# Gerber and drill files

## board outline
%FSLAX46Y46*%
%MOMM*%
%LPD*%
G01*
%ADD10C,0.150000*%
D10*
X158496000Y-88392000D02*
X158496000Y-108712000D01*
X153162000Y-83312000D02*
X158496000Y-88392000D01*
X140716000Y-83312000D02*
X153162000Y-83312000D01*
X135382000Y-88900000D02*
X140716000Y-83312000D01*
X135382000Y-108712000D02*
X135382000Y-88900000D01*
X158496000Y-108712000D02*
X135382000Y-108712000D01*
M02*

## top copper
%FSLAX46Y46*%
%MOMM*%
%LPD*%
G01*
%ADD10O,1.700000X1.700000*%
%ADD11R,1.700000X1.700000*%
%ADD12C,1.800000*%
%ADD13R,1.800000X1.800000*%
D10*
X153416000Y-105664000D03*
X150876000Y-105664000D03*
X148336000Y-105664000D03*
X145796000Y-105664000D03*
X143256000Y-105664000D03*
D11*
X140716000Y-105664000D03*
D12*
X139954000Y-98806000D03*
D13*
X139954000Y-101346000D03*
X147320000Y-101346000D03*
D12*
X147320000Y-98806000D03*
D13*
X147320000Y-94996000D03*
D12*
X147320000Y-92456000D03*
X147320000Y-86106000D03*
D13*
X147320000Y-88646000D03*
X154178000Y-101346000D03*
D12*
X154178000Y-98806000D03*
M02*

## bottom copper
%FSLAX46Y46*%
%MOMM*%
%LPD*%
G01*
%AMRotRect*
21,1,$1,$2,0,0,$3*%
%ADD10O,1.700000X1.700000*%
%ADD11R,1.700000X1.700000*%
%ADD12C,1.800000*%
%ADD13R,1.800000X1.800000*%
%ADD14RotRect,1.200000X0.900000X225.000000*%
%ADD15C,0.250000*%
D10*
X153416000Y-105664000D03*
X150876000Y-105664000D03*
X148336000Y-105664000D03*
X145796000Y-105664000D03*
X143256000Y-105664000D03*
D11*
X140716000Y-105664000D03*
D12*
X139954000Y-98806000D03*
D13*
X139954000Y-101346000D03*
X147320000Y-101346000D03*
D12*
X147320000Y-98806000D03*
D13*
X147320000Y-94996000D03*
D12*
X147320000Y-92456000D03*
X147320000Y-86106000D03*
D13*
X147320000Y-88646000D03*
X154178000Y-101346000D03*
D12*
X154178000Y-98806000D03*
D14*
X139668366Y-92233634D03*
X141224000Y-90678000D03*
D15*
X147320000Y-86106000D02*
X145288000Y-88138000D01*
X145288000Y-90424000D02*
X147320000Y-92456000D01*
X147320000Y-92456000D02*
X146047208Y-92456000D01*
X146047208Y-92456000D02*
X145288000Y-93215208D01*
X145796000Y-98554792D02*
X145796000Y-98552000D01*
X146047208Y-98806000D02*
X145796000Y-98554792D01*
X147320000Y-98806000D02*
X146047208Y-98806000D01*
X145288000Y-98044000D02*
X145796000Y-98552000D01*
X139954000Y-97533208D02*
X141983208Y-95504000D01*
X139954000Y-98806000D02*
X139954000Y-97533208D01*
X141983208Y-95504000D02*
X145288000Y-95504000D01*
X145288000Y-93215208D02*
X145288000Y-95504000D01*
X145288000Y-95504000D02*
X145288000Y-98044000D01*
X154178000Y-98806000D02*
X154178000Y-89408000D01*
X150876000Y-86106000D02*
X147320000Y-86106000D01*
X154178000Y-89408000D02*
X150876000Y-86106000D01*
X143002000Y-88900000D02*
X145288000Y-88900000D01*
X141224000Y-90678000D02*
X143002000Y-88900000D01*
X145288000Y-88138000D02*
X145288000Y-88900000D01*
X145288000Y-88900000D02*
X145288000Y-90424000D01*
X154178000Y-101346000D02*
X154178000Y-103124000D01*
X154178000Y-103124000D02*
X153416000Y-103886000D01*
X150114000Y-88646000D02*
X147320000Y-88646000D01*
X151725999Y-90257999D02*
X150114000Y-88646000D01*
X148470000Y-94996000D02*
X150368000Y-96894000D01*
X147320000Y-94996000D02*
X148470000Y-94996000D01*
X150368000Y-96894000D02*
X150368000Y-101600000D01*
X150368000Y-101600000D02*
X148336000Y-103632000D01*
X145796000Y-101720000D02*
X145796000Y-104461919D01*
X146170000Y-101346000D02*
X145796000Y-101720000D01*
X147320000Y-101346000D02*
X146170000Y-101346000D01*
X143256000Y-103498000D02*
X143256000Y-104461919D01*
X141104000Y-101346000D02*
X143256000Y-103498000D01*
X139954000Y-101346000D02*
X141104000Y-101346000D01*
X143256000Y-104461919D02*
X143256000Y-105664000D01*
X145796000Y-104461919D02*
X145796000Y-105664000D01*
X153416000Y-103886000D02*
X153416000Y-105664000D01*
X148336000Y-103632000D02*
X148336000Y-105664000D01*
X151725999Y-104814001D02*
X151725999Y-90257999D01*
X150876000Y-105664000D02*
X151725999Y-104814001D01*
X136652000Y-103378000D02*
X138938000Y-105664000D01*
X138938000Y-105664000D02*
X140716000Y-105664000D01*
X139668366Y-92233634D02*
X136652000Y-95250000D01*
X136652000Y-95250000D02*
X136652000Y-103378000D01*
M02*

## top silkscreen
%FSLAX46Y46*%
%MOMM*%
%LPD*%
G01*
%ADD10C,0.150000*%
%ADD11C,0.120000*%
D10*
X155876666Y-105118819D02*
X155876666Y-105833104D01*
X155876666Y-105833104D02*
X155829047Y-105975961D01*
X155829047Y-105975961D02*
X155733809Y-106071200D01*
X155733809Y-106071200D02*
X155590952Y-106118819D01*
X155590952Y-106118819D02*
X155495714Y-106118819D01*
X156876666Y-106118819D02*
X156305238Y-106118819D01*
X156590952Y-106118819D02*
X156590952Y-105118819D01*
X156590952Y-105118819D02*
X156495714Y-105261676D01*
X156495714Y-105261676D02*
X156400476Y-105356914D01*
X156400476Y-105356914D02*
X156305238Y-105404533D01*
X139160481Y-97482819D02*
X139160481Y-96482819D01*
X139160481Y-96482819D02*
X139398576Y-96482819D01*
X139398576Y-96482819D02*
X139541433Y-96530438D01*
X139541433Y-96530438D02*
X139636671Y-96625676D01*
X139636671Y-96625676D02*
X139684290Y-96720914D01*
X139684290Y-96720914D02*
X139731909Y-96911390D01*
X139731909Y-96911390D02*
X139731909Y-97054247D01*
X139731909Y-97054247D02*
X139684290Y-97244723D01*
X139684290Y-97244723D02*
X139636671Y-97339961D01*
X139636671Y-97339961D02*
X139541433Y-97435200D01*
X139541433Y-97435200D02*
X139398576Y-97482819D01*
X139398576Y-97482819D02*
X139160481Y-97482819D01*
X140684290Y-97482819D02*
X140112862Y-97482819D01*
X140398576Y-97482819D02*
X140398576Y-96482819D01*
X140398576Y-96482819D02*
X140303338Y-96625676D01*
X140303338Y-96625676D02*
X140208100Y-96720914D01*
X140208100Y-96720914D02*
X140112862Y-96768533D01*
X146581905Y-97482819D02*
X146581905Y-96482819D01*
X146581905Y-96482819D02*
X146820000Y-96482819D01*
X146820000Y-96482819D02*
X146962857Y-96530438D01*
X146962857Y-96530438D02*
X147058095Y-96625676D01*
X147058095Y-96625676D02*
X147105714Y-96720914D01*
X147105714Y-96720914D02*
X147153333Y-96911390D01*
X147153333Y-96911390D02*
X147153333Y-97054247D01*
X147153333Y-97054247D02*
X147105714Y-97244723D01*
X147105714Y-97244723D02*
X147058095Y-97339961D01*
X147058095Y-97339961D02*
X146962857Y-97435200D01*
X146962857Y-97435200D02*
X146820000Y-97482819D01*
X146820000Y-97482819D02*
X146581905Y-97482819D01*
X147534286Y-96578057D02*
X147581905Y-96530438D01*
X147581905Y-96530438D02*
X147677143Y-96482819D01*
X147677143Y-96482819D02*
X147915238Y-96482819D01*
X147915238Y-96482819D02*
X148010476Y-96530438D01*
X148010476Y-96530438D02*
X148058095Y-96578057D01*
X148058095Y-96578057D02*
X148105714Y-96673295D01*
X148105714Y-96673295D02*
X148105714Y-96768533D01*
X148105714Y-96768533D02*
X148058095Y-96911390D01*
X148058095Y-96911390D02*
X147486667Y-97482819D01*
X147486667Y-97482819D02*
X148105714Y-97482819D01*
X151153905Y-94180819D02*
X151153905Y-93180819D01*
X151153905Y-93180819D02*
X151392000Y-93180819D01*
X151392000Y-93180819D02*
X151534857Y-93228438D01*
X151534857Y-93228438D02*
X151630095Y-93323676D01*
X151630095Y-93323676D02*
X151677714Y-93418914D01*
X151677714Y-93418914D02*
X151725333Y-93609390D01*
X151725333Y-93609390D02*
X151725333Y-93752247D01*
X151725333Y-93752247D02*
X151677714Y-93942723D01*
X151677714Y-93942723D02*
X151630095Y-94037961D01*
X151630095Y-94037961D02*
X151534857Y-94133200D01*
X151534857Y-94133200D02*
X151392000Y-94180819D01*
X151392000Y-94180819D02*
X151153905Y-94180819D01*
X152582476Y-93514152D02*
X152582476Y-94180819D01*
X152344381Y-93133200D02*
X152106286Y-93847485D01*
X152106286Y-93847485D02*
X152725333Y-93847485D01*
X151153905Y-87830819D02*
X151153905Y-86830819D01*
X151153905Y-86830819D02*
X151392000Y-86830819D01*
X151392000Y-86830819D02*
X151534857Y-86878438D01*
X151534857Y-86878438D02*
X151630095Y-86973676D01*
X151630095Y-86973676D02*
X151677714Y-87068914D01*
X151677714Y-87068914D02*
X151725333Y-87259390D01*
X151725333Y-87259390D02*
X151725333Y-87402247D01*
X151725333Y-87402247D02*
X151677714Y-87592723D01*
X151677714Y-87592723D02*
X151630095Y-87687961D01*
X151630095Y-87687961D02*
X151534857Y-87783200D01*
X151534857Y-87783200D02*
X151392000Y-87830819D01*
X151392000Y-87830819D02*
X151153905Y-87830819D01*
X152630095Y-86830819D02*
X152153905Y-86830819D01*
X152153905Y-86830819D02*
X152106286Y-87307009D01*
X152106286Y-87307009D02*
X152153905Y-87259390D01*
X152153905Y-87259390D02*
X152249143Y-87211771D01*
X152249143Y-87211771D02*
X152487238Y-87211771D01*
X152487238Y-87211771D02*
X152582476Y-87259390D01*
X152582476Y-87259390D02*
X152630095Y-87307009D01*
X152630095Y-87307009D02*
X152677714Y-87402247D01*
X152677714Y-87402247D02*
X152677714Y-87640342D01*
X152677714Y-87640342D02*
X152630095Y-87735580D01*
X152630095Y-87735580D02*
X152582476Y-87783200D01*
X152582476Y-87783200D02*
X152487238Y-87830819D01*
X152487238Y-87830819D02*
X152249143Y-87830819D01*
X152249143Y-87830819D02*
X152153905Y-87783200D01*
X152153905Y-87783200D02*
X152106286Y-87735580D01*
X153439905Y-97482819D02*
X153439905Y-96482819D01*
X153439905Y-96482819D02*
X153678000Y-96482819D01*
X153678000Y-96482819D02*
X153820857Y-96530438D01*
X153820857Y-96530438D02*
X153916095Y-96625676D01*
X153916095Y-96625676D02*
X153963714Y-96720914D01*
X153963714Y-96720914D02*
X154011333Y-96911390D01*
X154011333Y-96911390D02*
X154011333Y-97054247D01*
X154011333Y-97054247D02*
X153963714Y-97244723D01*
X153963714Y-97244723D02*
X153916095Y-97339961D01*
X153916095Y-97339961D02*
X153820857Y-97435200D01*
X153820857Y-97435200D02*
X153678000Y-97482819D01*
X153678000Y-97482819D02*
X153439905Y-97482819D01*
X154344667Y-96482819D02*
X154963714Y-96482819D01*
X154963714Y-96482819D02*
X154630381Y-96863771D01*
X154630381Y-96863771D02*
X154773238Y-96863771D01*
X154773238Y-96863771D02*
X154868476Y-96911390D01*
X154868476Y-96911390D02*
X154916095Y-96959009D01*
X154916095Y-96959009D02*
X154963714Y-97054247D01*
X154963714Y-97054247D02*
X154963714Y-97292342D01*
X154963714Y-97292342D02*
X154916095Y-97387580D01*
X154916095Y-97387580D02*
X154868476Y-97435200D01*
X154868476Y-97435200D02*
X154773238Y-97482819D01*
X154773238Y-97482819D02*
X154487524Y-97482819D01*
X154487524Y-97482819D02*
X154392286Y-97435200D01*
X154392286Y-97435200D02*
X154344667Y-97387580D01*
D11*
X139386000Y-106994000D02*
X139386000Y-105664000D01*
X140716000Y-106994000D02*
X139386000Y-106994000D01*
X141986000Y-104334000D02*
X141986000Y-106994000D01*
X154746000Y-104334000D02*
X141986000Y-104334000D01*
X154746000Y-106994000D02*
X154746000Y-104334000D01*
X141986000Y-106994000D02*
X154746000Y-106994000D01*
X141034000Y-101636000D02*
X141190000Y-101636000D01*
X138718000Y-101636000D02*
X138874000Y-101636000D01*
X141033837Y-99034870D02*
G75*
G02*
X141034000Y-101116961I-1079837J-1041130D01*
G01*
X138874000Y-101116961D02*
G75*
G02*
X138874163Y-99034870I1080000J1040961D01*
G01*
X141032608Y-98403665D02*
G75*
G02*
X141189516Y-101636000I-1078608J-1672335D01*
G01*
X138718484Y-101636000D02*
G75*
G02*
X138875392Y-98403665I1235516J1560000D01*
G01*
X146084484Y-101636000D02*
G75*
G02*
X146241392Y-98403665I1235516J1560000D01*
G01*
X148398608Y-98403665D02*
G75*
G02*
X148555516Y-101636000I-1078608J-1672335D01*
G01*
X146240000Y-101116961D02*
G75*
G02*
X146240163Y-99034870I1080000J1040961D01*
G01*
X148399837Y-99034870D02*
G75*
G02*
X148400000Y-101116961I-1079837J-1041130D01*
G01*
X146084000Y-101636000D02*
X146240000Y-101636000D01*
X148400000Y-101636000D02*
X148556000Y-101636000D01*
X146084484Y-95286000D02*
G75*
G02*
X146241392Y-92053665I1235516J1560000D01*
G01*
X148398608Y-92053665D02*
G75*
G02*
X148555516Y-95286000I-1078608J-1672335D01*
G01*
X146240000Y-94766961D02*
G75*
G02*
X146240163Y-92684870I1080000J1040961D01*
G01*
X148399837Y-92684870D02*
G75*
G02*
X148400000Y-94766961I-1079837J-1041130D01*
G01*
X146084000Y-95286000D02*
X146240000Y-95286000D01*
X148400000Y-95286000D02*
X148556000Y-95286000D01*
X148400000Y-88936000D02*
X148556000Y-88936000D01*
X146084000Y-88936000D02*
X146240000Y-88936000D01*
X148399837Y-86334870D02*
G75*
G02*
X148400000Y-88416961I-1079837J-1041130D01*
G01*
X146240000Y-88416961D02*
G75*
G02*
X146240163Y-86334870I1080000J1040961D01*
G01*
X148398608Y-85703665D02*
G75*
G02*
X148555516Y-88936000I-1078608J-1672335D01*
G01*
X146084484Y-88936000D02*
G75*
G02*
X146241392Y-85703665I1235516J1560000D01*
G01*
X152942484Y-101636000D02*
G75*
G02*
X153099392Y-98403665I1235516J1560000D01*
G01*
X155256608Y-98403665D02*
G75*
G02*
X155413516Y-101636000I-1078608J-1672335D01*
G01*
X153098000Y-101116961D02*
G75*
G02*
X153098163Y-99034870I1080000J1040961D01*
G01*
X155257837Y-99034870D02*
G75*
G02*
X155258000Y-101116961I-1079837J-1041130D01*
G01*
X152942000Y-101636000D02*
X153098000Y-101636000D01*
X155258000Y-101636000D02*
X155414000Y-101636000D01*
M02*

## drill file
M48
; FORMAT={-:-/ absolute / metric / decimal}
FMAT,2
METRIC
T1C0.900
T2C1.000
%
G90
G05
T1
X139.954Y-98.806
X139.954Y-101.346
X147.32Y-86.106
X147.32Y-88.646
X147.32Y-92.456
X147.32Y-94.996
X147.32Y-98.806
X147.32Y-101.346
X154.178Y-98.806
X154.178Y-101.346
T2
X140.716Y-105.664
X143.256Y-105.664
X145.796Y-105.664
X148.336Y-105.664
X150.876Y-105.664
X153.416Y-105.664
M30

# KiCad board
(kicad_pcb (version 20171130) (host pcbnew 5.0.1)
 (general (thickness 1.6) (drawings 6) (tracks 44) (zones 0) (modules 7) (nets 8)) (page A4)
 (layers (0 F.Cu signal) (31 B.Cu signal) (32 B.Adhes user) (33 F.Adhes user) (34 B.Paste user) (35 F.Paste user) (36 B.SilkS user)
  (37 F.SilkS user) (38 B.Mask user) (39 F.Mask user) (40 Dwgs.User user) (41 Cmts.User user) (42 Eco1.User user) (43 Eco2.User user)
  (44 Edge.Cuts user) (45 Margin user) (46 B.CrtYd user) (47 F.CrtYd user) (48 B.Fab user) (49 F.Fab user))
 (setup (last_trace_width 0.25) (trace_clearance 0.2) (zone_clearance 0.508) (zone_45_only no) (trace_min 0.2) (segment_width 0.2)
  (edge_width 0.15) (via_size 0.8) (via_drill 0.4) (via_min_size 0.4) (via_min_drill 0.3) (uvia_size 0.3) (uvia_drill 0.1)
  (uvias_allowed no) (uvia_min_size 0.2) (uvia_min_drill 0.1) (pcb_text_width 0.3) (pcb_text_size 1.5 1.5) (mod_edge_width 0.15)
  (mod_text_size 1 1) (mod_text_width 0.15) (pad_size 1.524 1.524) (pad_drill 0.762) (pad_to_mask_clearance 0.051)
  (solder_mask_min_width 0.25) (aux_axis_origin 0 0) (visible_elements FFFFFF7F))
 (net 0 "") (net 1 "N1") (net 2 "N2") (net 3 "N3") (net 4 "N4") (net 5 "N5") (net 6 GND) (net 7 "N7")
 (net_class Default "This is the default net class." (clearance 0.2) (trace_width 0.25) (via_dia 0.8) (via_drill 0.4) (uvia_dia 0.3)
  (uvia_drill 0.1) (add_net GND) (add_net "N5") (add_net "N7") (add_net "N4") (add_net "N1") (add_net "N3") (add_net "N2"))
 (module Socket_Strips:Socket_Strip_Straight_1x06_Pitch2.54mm (layer F.Cu) (at 140.716 105.664 90)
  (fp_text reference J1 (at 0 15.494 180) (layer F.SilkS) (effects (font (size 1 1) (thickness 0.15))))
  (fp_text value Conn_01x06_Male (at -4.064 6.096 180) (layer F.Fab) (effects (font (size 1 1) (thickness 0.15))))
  (fp_line (start -1.33 -1.33) (end 0 -1.33) (layer F.SilkS) (width 0.12))
  (fp_line (start -1.33 0) (end -1.33 -1.33) (layer F.SilkS) (width 0.12))
  (fp_line (start 1.33 1.27) (end -1.33 1.27) (layer F.SilkS) (width 0.12))
  (fp_line (start 1.33 14.03) (end 1.33 1.27) (layer F.SilkS) (width 0.12))
  (fp_line (start -1.33 14.03) (end 1.33 14.03) (layer F.SilkS) (width 0.12))
  (fp_line (start -1.33 1.27) (end -1.33 14.03) (layer F.SilkS) (width 0.12))
  (pad 6 thru_hole oval (at 0 12.7 90) (size 1.7 1.7) (drill 1) (layers *.Cu *.Mask) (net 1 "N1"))
  (pad 5 thru_hole oval (at 0 10.16 90) (size 1.7 1.7) (drill 1) (layers *.Cu *.Mask) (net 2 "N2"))
  (pad 4 thru_hole oval (at 0 7.62 90) (size 1.7 1.7) (drill 1) (layers *.Cu *.Mask) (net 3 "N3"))
  (pad 3 thru_hole oval (at 0 5.08 90) (size 1.7 1.7) (drill 1) (layers *.Cu *.Mask) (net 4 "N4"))
  (pad 2 thru_hole oval (at 0 2.54 90) (size 1.7 1.7) (drill 1) (layers *.Cu *.Mask) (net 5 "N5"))
  (pad 1 thru_hole rect (at 0 0 90) (size 1.7 1.7) (drill 1) (layers *.Cu *.Mask) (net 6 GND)))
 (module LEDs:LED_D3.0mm (layer F.Cu) (at 139.954 101.346 90)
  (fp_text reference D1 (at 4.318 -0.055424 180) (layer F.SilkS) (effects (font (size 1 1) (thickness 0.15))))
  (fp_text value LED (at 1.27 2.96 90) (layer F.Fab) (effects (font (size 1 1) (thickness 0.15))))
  (fp_line (start -0.29 1.08) (end -0.29 1.236) (layer F.SilkS) (width 0.12))
  (fp_line (start -0.29 -1.236) (end -0.29 -1.08) (layer F.SilkS) (width 0.12))
  (fp_arc (start 1.27 0) (end 0.229039 1.08) (angle -87.9) (layer F.SilkS) (width 0.12))
  (fp_arc (start 1.27 0) (end 0.229039 -1.08) (angle 87.9) (layer F.SilkS) (width 0.12))
  (fp_arc (start 1.27 0) (end -0.29 1.235516) (angle -108.8) (layer F.SilkS) (width 0.12))
  (fp_arc (start 1.27 0) (end -0.29 -1.235516) (angle 108.8) (layer F.SilkS) (width 0.12))
  (pad 2 thru_hole circle (at 2.54 0 90) (size 1.8 1.8) (drill 0.9) (layers *.Cu *.Mask) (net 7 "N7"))
  (pad 1 thru_hole rect (at 0 0 90) (size 1.8 1.8) (drill 0.9) (layers *.Cu *.Mask) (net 5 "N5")))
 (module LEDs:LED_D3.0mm (layer F.Cu) (at 147.32 101.346 90)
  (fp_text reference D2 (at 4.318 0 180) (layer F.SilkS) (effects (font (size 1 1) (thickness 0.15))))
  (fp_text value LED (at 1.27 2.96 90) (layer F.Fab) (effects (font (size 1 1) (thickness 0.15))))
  (fp_arc (start 1.27 0) (end -0.29 -1.235516) (angle 108.8) (layer F.SilkS) (width 0.12))
  (fp_arc (start 1.27 0) (end -0.29 1.235516) (angle -108.8) (layer F.SilkS) (width 0.12))
  (fp_arc (start 1.27 0) (end 0.229039 -1.08) (angle 87.9) (layer F.SilkS) (width 0.12))
  (fp_arc (start 1.27 0) (end 0.229039 1.08) (angle -87.9) (layer F.SilkS) (width 0.12))
  (fp_line (start -0.29 -1.236) (end -0.29 -1.08) (layer F.SilkS) (width 0.12))
  (fp_line (start -0.29 1.08) (end -0.29 1.236) (layer F.SilkS) (width 0.12))
  (pad 1 thru_hole rect (at 0 0 90) (size 1.8 1.8) (drill 0.9) (layers *.Cu *.Mask) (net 4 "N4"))
  (pad 2 thru_hole circle (at 2.54 0 90) (size 1.8 1.8) (drill 0.9) (layers *.Cu *.Mask) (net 7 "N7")))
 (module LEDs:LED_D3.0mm (layer F.Cu) (at 147.32 94.996 90)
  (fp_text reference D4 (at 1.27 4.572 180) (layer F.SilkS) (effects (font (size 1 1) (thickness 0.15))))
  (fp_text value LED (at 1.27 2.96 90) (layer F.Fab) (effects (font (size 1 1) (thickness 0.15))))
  (fp_arc (start 1.27 0) (end -0.29 -1.235516) (angle 108.8) (layer F.SilkS) (width 0.12))
  (fp_arc (start 1.27 0) (end -0.29 1.235516) (angle -108.8) (layer F.SilkS) (width 0.12))
  (fp_arc (start 1.27 0) (end 0.229039 -1.08) (angle 87.9) (layer F.SilkS) (width 0.12))
  (fp_arc (start 1.27 0) (end 0.229039 1.08) (angle -87.9) (layer F.SilkS) (width 0.12))
  (fp_line (start -0.29 -1.236) (end -0.29 -1.08) (layer F.SilkS) (width 0.12))
  (fp_line (start -0.29 1.08) (end -0.29 1.236) (layer F.SilkS) (width 0.12))
  (pad 1 thru_hole rect (at 0 0 90) (size 1.8 1.8) (drill 0.9) (layers *.Cu *.Mask) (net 3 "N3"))
  (pad 2 thru_hole circle (at 2.54 0 90) (size 1.8 1.8) (drill 0.9) (layers *.Cu *.Mask) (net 7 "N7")))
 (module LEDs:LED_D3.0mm (layer F.Cu) (at 147.32 88.646 90)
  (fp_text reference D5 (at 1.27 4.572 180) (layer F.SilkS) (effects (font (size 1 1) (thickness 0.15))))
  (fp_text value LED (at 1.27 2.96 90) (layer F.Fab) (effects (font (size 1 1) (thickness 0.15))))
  (fp_line (start -0.29 1.08) (end -0.29 1.236) (layer F.SilkS) (width 0.12))
  (fp_line (start -0.29 -1.236) (end -0.29 -1.08) (layer F.SilkS) (width 0.12))
  (fp_arc (start 1.27 0) (end 0.229039 1.08) (angle -87.9) (layer F.SilkS) (width 0.12))
  (fp_arc (start 1.27 0) (end 0.229039 -1.08) (angle 87.9) (layer F.SilkS) (width 0.12))
  (fp_arc (start 1.27 0) (end -0.29 1.235516) (angle -108.8) (layer F.SilkS) (width 0.12))
  (fp_arc (start 1.27 0) (end -0.29 -1.235516) (angle 108.8) (layer F.SilkS) (width 0.12))
  (pad 2 thru_hole circle (at 2.54 0 90) (size 1.8 1.8) (drill 0.9) (layers *.Cu *.Mask) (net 7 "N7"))
  (pad 1 thru_hole rect (at 0 0 90) (size 1.8 1.8) (drill 0.9) (layers *.Cu *.Mask) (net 2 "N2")))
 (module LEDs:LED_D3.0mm (layer F.Cu) (at 154.178 101.346 90)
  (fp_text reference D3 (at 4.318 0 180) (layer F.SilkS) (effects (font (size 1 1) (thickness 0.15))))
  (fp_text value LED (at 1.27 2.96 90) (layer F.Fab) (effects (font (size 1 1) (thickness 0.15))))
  (fp_arc (start 1.27 0) (end -0.29 -1.235516) (angle 108.8) (layer F.SilkS) (width 0.12))
  (fp_arc (start 1.27 0) (end -0.29 1.235516) (angle -108.8) (layer F.SilkS) (width 0.12))
  (fp_arc (start 1.27 0) (end 0.229039 -1.08) (angle 87.9) (layer F.SilkS) (width 0.12))
  (fp_arc (start 1.27 0) (end 0.229039 1.08) (angle -87.9) (layer F.SilkS) (width 0.12))
  (fp_line (start -0.29 -1.236) (end -0.29 -1.08) (layer F.SilkS) (width 0.12))
  (fp_line (start -0.29 1.08) (end -0.29 1.236) (layer F.SilkS) (width 0.12))
  (pad 1 thru_hole rect (at 0 0 90) (size 1.8 1.8) (drill 0.9) (layers *.Cu *.Mask) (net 1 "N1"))
  (pad 2 thru_hole circle (at 2.54 0 90) (size 1.8 1.8) (drill 0.9) (layers *.Cu *.Mask) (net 7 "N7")))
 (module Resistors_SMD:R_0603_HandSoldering (layer B.Cu) (at 140.446183 91.455817 225)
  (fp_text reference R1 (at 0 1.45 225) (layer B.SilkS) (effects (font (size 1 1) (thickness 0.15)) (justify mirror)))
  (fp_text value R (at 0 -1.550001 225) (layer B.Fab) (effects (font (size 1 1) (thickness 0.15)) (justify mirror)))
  (pad 2 smd rect (at 1.099999 0 225) (size 1.2 0.9) (layers B.Cu B.Paste B.Mask) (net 6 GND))
  (pad 1 smd rect (at -1.099999 0 225) (size 1.2 0.9) (layers B.Cu B.Paste B.Mask) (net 7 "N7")))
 (gr_line (start 158.496 88.392) (end 158.496 108.712) (layer Edge.Cuts) (width 0.15))
 (gr_line (start 153.162 83.312) (end 158.496 88.392) (layer Edge.Cuts) (width 0.15))
 (gr_line (start 140.716 83.312) (end 153.162 83.312) (layer Edge.Cuts) (width 0.15))
 (gr_line (start 135.382 88.9) (end 140.716 83.312) (layer Edge.Cuts) (width 0.15))
 (gr_line (start 135.382 108.712) (end 135.382 88.9) (layer Edge.Cuts) (width 0.15))
 (gr_line (start 158.496 108.712) (end 135.382 108.712) (layer Edge.Cuts) (width 0.15))
 (segment (start 147.32 86.106) (end 145.288 88.138) (width 0.25) (layer B.Cu) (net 7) (status 10))
 (segment (start 145.288 90.424) (end 147.32 92.456) (width 0.25) (layer B.Cu) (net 7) (status 20))
 (segment (start 147.32 92.456) (end 146.047208 92.456) (width 0.25) (layer B.Cu) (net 7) (status 10))
 (segment (start 146.047208 92.456) (end 145.288 93.215208) (width 0.25) (layer B.Cu) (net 7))
 (segment (start 145.796 98.554792) (end 145.796 98.552) (width 0.25) (layer B.Cu) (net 7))
 (segment (start 146.047208 98.806) (end 145.796 98.554792) (width 0.25) (layer B.Cu) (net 7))
 (segment (start 147.32 98.806) (end 146.047208 98.806) (width 0.25) (layer B.Cu) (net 7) (status 10))
 (segment (start 145.288 98.044) (end 145.796 98.552) (width 0.25) (layer B.Cu) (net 7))
 (segment (start 139.954 97.533208) (end 141.983208 95.504) (width 0.25) (layer B.Cu) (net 7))
 (segment (start 139.954 98.806) (end 139.954 97.533208) (width 0.25) (layer B.Cu) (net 7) (status 10))
 (segment (start 141.983208 95.504) (end 145.288 95.504) (width 0.25) (layer B.Cu) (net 7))
 (segment (start 145.288 93.215208) (end 145.288 95.504) (width 0.25) (layer B.Cu) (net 7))
 (segment (start 145.288 95.504) (end 145.288 98.044) (width 0.25) (layer B.Cu) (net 7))
 (segment (start 154.178 98.806) (end 154.178 89.408) (width 0.25) (layer B.Cu) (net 7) (status 10))
 (segment (start 150.876 86.106) (end 147.32 86.106) (width 0.25) (layer B.Cu) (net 7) (status 20))
 (segment (start 154.178 89.408) (end 150.876 86.106) (width 0.25) (layer B.Cu) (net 7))
 (segment (start 143.002 88.9) (end 145.288 88.9) (width 0.25) (layer B.Cu) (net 7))
 (segment (start 141.224 90.678) (end 143.002 88.9) (width 0.25) (layer B.Cu) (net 7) (status 10))
 (segment (start 145.288 88.138) (end 145.288 88.9) (width 0.25) (layer B.Cu) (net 7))
 (segment (start 145.288 88.9) (end 145.288 90.424) (width 0.25) (layer B.Cu) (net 7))
 (segment (start 154.178 101.346) (end 154.178 103.124) (width 0.25) (layer B.Cu) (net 1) (status 10))
 (segment (start 154.178 103.124) (end 153.416 103.886) (width 0.25) (layer B.Cu) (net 1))
 (segment (start 150.114 88.646) (end 147.32 88.646) (width 0.25) (layer B.Cu) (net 2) (status 20))
 (segment (start 151.725999 90.257999) (end 150.114 88.646) (width 0.25) (layer B.Cu) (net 2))
 (segment (start 148.47 94.996) (end 150.368 96.894) (width 0.25) (layer B.Cu) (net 3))
 (segment (start 147.32 94.996) (end 148.47 94.996) (width 0.25) (layer B.Cu) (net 3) (status 10))
 (segment (start 150.368 96.894) (end 150.368 101.6) (width 0.25) (layer B.Cu) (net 3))
 (segment (start 150.368 101.6) (end 148.336 103.632) (width 0.25) (layer B.Cu) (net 3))
 (segment (start 145.796 101.72) (end 145.796 104.461919) (width 0.25) (layer B.Cu) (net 4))
 (segment (start 146.17 101.346) (end 145.796 101.72) (width 0.25) (layer B.Cu) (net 4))
 (segment (start 147.32 101.346) (end 146.17 101.346) (width 0.25) (layer B.Cu) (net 4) (status 10))
 (segment (start 143.256 103.498) (end 143.256 104.461919) (width 0.25) (layer B.Cu) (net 5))
 (segment (start 141.104 101.346) (end 143.256 103.498) (width 0.25) (layer B.Cu) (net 5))
 (segment (start 139.954 101.346) (end 141.104 101.346) (width 0.25) (layer B.Cu) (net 5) (status 10))
 (segment (start 143.256 104.461919) (end 143.256 105.664) (width 0.25) (layer B.Cu) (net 5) (status 20))
 (segment (start 145.796 104.461919) (end 145.796 105.664) (width 0.25) (layer B.Cu) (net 4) (status 20))
 (segment (start 153.416 103.886) (end 153.416 105.664) (width 0.25) (layer B.Cu) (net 1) (status 20))
 (segment (start 148.336 103.632) (end 148.336 105.664) (width 0.25) (layer B.Cu) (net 3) (status 20))
 (segment (start 151.725999 104.814001) (end 151.725999 90.257999) (width 0.25) (layer B.Cu) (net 2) (status 10))
 (segment (start 150.876 105.664) (end 151.725999 104.814001) (width 0.25) (layer B.Cu) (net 2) (status 30))
 (segment (start 136.652 103.378) (end 138.938 105.664) (width 0.25) (layer B.Cu) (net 6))
 (segment (start 138.938 105.664) (end 140.716 105.664) (width 0.25) (layer B.Cu) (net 6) (status 20))
 (segment (start 139.668366 92.233634) (end 136.652 95.25) (width 0.25) (layer B.Cu) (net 6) (status 10))
 (segment (start 136.652 95.25) (end 136.652 103.378) (width 0.25) (layer B.Cu) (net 6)))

